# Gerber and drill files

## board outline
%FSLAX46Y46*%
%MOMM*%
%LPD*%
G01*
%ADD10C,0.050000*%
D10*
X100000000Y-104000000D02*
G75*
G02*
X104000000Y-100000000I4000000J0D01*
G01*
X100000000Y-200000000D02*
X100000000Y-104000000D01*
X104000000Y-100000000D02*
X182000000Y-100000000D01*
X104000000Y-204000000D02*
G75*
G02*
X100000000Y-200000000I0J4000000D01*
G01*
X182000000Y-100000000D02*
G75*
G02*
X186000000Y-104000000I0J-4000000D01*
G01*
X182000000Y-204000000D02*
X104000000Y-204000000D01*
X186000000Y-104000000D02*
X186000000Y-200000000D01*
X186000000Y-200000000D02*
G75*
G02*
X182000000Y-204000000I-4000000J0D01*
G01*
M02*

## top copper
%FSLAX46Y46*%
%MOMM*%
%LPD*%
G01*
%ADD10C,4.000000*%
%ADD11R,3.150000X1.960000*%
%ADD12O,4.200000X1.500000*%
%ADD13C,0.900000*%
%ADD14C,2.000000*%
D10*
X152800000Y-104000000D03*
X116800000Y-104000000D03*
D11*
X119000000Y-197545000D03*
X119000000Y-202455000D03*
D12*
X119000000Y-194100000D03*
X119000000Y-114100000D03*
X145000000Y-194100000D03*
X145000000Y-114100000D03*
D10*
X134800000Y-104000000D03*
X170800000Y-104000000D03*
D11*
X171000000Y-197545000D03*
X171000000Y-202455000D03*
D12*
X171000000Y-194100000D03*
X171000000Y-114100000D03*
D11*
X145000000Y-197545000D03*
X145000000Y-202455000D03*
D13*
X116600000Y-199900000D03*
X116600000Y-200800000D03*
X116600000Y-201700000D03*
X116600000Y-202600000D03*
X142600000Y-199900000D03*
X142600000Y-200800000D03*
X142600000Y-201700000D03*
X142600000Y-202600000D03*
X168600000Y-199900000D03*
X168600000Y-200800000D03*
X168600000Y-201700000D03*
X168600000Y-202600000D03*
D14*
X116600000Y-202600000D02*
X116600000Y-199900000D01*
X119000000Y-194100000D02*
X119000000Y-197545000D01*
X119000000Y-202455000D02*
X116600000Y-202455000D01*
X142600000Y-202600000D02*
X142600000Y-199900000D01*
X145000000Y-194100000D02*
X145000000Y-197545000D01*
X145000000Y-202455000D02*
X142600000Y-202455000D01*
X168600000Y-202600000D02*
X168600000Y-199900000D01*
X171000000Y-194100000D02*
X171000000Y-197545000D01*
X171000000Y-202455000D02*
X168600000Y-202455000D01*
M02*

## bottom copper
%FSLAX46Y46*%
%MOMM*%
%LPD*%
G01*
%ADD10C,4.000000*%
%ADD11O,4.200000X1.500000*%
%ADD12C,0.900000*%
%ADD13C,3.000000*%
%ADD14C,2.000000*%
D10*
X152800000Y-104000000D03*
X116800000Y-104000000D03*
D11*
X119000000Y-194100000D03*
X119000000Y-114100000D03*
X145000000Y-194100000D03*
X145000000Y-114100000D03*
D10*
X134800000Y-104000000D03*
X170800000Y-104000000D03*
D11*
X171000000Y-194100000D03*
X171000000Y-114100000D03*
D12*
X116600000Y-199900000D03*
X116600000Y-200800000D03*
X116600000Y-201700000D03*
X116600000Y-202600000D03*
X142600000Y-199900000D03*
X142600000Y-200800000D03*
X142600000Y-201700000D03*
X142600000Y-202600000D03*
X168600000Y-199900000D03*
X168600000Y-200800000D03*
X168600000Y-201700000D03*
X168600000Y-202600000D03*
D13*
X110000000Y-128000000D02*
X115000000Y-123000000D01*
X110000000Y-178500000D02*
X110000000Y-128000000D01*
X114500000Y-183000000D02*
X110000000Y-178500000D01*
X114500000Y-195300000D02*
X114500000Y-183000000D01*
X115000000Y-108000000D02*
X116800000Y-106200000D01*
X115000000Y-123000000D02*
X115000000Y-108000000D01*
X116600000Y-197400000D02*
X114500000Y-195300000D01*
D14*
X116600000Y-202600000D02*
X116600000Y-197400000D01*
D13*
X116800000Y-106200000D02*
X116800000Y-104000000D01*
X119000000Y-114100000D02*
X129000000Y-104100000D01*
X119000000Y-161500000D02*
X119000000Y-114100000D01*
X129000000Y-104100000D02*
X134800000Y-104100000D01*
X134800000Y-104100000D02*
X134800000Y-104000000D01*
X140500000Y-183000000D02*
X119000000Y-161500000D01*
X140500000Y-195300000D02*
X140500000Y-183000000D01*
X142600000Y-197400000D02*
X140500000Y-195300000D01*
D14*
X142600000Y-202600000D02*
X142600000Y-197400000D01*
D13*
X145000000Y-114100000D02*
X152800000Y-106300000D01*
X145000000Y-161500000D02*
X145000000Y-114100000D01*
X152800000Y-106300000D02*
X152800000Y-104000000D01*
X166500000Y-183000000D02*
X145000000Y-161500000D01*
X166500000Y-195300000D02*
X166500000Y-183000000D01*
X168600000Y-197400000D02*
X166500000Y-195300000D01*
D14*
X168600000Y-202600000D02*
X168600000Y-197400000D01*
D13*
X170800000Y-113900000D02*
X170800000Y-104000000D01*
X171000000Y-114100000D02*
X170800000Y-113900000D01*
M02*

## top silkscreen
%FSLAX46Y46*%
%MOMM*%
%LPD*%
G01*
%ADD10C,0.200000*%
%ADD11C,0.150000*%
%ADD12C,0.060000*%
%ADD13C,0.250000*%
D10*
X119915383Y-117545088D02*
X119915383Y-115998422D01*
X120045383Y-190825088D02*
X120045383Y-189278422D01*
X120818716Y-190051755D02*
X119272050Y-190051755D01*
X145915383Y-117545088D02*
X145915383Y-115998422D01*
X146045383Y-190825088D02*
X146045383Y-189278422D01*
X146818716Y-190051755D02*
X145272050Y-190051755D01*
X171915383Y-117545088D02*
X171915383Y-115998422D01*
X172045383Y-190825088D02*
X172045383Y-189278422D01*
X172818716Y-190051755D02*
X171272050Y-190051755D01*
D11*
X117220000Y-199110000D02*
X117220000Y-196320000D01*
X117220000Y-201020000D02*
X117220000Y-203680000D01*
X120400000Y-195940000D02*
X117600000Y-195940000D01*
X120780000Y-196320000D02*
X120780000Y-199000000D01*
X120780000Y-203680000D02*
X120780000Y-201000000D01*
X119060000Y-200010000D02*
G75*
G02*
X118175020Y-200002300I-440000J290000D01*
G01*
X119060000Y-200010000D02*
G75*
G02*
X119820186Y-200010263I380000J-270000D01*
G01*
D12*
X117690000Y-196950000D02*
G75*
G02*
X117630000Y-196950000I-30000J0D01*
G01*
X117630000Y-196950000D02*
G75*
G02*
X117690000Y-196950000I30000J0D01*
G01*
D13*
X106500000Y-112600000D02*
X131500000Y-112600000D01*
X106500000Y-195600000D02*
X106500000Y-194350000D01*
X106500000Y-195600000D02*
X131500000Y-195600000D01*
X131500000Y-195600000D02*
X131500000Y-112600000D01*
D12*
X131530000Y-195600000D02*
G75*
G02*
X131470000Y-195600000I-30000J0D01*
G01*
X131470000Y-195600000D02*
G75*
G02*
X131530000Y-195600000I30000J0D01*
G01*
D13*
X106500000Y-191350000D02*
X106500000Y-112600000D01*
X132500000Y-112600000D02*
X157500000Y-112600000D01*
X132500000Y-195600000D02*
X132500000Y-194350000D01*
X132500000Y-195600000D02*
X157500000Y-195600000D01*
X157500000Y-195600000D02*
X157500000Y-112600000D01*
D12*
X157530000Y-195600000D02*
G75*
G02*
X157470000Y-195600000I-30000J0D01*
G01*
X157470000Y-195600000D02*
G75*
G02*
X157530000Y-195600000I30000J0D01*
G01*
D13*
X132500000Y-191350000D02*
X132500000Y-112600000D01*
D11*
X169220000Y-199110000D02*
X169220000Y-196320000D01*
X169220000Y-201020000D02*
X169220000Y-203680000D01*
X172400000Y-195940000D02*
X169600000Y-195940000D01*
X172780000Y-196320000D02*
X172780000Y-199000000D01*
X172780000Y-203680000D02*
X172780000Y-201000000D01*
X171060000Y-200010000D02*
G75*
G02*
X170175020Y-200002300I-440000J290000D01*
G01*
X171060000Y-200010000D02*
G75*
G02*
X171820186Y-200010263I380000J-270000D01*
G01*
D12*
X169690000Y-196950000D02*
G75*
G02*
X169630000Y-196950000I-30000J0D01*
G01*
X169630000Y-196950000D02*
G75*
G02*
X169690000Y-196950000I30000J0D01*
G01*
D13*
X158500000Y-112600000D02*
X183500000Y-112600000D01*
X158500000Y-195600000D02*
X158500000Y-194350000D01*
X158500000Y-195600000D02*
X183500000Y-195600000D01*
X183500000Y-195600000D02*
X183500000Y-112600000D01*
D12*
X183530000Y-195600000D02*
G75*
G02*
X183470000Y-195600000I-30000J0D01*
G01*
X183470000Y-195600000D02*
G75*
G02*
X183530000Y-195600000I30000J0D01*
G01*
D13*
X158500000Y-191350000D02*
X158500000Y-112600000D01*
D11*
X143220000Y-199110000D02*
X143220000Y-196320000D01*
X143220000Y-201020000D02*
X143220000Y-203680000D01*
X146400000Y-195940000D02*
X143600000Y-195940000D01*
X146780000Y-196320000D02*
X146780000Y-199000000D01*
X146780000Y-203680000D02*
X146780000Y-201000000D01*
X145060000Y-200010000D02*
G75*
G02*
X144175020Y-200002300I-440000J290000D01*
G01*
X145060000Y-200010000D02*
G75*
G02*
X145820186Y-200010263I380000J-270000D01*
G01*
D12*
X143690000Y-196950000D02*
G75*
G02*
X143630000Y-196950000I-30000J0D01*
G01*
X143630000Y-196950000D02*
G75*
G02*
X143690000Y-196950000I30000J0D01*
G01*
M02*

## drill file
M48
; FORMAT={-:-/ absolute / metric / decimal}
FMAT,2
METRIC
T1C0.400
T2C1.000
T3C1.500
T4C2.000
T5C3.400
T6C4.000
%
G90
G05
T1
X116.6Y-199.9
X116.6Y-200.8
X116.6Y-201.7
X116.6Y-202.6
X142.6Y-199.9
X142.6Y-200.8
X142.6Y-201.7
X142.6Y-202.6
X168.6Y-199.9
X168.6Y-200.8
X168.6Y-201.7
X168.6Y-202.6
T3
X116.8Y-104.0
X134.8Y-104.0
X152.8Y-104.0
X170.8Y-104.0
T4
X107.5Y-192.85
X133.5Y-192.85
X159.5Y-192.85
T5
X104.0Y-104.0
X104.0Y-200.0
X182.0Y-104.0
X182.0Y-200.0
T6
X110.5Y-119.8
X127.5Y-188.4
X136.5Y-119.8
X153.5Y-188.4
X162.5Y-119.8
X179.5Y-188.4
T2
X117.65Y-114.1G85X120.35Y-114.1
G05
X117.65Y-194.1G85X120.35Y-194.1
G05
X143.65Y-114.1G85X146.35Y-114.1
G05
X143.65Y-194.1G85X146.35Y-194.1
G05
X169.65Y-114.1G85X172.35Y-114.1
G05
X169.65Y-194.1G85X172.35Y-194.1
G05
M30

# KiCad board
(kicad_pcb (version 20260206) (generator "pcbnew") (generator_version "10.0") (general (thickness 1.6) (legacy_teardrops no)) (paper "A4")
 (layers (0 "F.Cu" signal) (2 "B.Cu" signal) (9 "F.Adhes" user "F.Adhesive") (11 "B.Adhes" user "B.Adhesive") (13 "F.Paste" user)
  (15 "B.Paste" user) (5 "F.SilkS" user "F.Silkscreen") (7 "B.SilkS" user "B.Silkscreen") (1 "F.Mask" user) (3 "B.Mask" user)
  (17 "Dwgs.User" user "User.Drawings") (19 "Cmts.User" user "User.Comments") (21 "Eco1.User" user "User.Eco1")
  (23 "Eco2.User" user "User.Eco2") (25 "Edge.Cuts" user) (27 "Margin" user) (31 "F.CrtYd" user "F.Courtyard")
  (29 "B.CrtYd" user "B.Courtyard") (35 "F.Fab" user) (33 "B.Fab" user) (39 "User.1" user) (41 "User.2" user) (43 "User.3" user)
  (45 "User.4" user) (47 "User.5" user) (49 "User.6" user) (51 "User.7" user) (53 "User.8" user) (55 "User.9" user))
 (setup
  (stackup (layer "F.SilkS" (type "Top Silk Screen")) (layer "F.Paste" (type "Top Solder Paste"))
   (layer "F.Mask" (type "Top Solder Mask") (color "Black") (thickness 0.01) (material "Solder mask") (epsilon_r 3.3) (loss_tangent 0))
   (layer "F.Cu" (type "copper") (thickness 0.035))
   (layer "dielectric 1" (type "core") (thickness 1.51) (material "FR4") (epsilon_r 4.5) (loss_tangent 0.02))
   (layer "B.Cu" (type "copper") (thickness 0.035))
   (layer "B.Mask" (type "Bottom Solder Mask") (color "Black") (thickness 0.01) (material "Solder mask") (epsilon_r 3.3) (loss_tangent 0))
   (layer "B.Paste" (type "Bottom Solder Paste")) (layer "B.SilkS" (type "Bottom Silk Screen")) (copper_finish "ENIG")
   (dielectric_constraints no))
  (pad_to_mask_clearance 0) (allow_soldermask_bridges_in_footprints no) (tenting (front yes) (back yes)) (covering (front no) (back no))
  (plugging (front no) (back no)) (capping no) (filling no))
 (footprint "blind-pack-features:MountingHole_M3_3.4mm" (layer "F.Cu") (at 182 200)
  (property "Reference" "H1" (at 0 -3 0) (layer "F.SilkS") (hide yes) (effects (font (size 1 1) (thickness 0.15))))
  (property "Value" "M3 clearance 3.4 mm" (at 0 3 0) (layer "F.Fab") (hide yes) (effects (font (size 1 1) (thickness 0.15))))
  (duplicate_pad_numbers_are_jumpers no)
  (pad "" np_thru_hole circle (at 0 0) (size 3.4 3.4) (drill 3.4) (layers "*.Cu" "*.Mask")))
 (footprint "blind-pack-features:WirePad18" (layer "F.Cu") (at 152.8 104)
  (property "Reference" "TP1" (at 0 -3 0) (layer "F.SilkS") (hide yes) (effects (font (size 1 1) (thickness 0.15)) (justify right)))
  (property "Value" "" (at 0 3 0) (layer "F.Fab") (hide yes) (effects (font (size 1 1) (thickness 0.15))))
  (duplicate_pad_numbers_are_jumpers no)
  (pad "1" thru_hole circle (at 0 0) (size 4 4) (drill 1.5) (layers "*.Cu" "*.Mask") (remove_unused_layers no) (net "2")))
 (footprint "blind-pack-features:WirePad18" (layer "F.Cu") (at 116.8 104)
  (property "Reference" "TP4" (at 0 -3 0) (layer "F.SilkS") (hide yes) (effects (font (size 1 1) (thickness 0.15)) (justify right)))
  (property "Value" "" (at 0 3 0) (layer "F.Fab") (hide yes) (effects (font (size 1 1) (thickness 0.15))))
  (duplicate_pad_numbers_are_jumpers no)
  (pad "1" thru_hole circle (at 0 0) (size 4 4) (drill 1.5) (layers "*.Cu" "*.Mask") (remove_unused_layers no) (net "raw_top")))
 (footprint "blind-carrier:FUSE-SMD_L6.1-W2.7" (layer "F.Cu") (at 119 200 -90)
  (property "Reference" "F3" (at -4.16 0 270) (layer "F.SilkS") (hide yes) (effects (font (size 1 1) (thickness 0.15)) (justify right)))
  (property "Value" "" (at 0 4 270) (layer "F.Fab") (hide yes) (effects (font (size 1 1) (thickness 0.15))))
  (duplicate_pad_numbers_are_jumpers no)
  (fp_line (start -0.89 1.78) (end -3.68 1.78) (stroke (width 0.15) (type solid)) (layer "F.SilkS"))
  (fp_line (start 1.02 1.78) (end 3.68 1.78) (stroke (width 0.15) (type solid)) (layer "F.SilkS"))
  (fp_line (start -4.06 -1.4) (end -4.06 1.4) (stroke (width 0.15) (type solid)) (layer "F.SilkS"))
  (fp_line (start -3.68 -1.78) (end -1 -1.78) (stroke (width 0.15) (type solid)) (layer "F.SilkS"))
  (fp_line (start 3.68 -1.78) (end 1 -1.78) (stroke (width 0.15) (type solid)) (layer "F.SilkS"))
  (fp_arc (start 0.01 -0.06) (mid 0.246953 0.384585) (end 0.0023 0.82498) (stroke (width 0.15) (type solid)) (layer "F.SilkS"))
  (fp_arc (start 0.01 -0.06) (mid -0.186154 -0.440161) (end 0.010263 -0.820186) (stroke (width 0.15) (type solid)) (layer "F.SilkS"))
  (fp_circle (center -3.05 1.34) (end -3.02 1.34) (stroke (width 0.06) (type solid)) (fill no) (layer "F.SilkS"))
  (pad "1" smd rect (at -2.455 0 270) (size 1.96 3.15) (layers "F.Cu" "F.Mask" "F.Paste") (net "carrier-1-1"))
  (pad "2" smd rect (at 2.455 0 270) (size 1.96 3.15) (layers "F.Cu" "F.Mask" "F.Paste") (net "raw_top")))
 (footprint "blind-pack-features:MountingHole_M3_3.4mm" (layer "F.Cu") (at 104 200)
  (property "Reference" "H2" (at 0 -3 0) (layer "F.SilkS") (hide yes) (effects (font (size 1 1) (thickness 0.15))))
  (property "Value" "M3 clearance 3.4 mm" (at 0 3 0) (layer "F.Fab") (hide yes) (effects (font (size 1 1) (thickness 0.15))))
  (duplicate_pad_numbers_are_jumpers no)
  (pad "" np_thru_hole circle (at 0 0) (size 3.4 3.4) (drill 3.4) (layers "*.Cu" "*.Mask")))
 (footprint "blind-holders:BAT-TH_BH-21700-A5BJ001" (layer "F.Cu") (at 119 154.1 90)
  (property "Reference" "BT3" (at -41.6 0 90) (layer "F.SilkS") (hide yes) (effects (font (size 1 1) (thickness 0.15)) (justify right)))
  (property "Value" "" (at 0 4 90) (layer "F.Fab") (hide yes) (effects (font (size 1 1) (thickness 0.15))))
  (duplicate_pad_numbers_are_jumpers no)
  (fp_line (start 41.5 -12.5) (end 41.5 12.5) (stroke (width 0.25) (type solid)) (layer "F.SilkS"))
  (fp_line (start -41.5 -12.5) (end -40.25 -12.5) (stroke (width 0.25) (type solid)) (layer "F.SilkS"))
  (fp_line (start -41.5 -12.5) (end -41.5 12.5) (stroke (width 0.25) (type solid)) (layer "F.SilkS"))
  (fp_line (start -41.5 12.5) (end 41.5 12.5) (stroke (width 0.25) (type solid)) (layer "F.SilkS"))
  (fp_circle (center -41.5 12.5) (end -41.47 12.5) (stroke (width 0.06) (type solid)) (fill no) (layer "F.SilkS"))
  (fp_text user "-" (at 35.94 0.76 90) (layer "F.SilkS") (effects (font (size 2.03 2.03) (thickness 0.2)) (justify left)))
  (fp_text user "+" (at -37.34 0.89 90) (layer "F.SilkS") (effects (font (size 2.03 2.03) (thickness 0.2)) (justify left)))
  (pad "" np_thru_hole circle (at -38.75 -11.5 90) (size 2 2) (drill 2) (layers "*.Cu" "*.Mask"))
  (pad "" np_thru_hole circle (at -34.3 8.5 90) (size 4 4) (drill 4) (layers "*.Cu" "*.Mask"))
  (pad "" np_thru_hole circle (at 34.3 -8.5 90) (size 4 4) (drill 4) (layers "*.Cu" "*.Mask"))
  (pad "1" thru_hole oval (at -40 0 90) (size 1.5 4.2) (drill oval 1 3.7) (layers "*.Cu" "*.Mask") (remove_unused_layers no)
   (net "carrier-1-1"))
  (pad "2" thru_hole oval (at 40 0 90) (size 1.5 4.2) (drill oval 1 3.7) (layers "*.Cu" "*.Mask") (remove_unused_layers no)
   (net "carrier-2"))
  (fp_line (start -37.25 -12.5) (end 41.5 -12.5) (stroke (width 0.25) (type solid)) (layer "F.SilkS")))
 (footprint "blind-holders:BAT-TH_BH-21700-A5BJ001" (layer "F.Cu") (at 145 154.1 90)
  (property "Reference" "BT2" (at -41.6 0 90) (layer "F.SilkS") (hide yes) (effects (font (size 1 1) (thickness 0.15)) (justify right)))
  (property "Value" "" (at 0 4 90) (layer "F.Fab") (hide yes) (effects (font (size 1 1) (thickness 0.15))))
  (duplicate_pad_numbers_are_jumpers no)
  (fp_line (start 41.5 -12.5) (end 41.5 12.5) (stroke (width 0.25) (type solid)) (layer "F.SilkS"))
  (fp_line (start -41.5 -12.5) (end -40.25 -12.5) (stroke (width 0.25) (type solid)) (layer "F.SilkS"))
  (fp_line (start -41.5 -12.5) (end -41.5 12.5) (stroke (width 0.25) (type solid)) (layer "F.SilkS"))
  (fp_line (start -41.5 12.5) (end 41.5 12.5) (stroke (width 0.25) (type solid)) (layer "F.SilkS"))
  (fp_circle (center -41.5 12.5) (end -41.47 12.5) (stroke (width 0.06) (type solid)) (fill no) (layer "F.SilkS"))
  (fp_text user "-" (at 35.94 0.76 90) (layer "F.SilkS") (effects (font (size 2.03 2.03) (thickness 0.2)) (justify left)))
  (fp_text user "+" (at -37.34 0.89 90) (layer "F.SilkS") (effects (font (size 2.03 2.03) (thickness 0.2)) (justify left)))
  (pad "" np_thru_hole circle (at -38.75 -11.5 90) (size 2 2) (drill 2) (layers "*.Cu" "*.Mask"))
  (pad "" np_thru_hole circle (at -34.3 8.5 90) (size 4 4) (drill 4) (layers "*.Cu" "*.Mask"))
  (pad "" np_thru_hole circle (at 34.3 -8.5 90) (size 4 4) (drill 4) (layers "*.Cu" "*.Mask"))
  (pad "1" thru_hole oval (at -40 0 90) (size 1.5 4.2) (drill oval 1 3.7) (layers "*.Cu" "*.Mask") (remove_unused_layers no)
   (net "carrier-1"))
  (pad "2" thru_hole oval (at 40 0 90) (size 1.5 4.2) (drill oval 1 3.7) (layers "*.Cu" "*.Mask") (remove_unused_layers no) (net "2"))
  (fp_line (start -37.25 -12.5) (end 41.5 -12.5) (stroke (width 0.25) (type solid)) (layer "F.SilkS")))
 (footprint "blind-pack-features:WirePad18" (layer "F.Cu") (at 134.8 104)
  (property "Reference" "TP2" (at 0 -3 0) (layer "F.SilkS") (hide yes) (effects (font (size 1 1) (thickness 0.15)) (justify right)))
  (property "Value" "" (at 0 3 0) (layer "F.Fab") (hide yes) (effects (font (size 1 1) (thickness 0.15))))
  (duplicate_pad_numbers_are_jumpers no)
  (pad "1" thru_hole circle (at 0 0) (size 4 4) (drill 1.5) (layers "*.Cu" "*.Mask") (remove_unused_layers no) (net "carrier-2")))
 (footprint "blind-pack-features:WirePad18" (layer "F.Cu") (at 170.8 104)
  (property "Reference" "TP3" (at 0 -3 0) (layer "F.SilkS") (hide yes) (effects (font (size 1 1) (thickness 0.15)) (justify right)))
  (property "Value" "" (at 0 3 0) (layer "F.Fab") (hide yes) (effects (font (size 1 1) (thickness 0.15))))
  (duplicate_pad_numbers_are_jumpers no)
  (pad "1" thru_hole circle (at 0 0) (size 4 4) (drill 1.5) (layers "*.Cu" "*.Mask") (remove_unused_layers no) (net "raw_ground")))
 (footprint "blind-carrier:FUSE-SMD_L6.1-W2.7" (layer "F.Cu") (at 171 200 -90)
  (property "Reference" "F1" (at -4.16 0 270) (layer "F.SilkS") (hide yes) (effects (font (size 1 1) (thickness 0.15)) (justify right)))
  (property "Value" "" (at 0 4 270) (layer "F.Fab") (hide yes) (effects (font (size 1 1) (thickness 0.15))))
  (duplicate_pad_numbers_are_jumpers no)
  (fp_line (start -0.89 1.78) (end -3.68 1.78) (stroke (width 0.15) (type solid)) (layer "F.SilkS"))
  (fp_line (start 1.02 1.78) (end 3.68 1.78) (stroke (width 0.15) (type solid)) (layer "F.SilkS"))
  (fp_line (start -4.06 -1.4) (end -4.06 1.4) (stroke (width 0.15) (type solid)) (layer "F.SilkS"))
  (fp_line (start -3.68 -1.78) (end -1 -1.78) (stroke (width 0.15) (type solid)) (layer "F.SilkS"))
  (fp_line (start 3.68 -1.78) (end 1 -1.78) (stroke (width 0.15) (type solid)) (layer "F.SilkS"))
  (fp_arc (start 0.01 -0.06) (mid 0.246953 0.384585) (end 0.0023 0.82498) (stroke (width 0.15) (type solid)) (layer "F.SilkS"))
  (fp_arc (start 0.01 -0.06) (mid -0.186154 -0.440161) (end 0.010263 -0.820186) (stroke (width 0.15) (type solid)) (layer "F.SilkS"))
  (fp_circle (center -3.05 1.34) (end -3.02 1.34) (stroke (width 0.06) (type solid)) (fill no) (layer "F.SilkS"))
  (pad "1" smd rect (at -2.455 0 270) (size 1.96 3.15) (layers "F.Cu" "F.Mask" "F.Paste") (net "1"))
  (pad "2" smd rect (at 2.455 0 270) (size 1.96 3.15) (layers "F.Cu" "F.Mask" "F.Paste") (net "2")))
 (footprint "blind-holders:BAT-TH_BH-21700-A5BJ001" (layer "F.Cu") (at 171 154.1 90)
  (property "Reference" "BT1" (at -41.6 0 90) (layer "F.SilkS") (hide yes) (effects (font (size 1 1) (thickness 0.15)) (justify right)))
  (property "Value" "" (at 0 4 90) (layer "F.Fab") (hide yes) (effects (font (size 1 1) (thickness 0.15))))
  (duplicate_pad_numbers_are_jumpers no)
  (fp_line (start 41.5 -12.5) (end 41.5 12.5) (stroke (width 0.25) (type solid)) (layer "F.SilkS"))
  (fp_line (start -41.5 -12.5) (end -40.25 -12.5) (stroke (width 0.25) (type solid)) (layer "F.SilkS"))
  (fp_line (start -41.5 -12.5) (end -41.5 12.5) (stroke (width 0.25) (type solid)) (layer "F.SilkS"))
  (fp_line (start -41.5 12.5) (end 41.5 12.5) (stroke (width 0.25) (type solid)) (layer "F.SilkS"))
  (fp_circle (center -41.5 12.5) (end -41.47 12.5) (stroke (width 0.06) (type solid)) (fill no) (layer "F.SilkS"))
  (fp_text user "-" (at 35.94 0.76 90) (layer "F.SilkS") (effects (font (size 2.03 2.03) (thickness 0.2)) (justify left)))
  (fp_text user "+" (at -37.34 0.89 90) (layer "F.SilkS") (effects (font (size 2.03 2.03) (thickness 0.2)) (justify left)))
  (pad "" np_thru_hole circle (at -38.75 -11.5 90) (size 2 2) (drill 2) (layers "*.Cu" "*.Mask"))
  (pad "" np_thru_hole circle (at -34.3 8.5 90) (size 4 4) (drill 4) (layers "*.Cu" "*.Mask"))
  (pad "" np_thru_hole circle (at 34.3 -8.5 90) (size 4 4) (drill 4) (layers "*.Cu" "*.Mask"))
  (pad "1" thru_hole oval (at -40 0 90) (size 1.5 4.2) (drill oval 1 3.7) (layers "*.Cu" "*.Mask") (remove_unused_layers no) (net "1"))
  (pad "2" thru_hole oval (at 40 0 90) (size 1.5 4.2) (drill oval 1 3.7) (layers "*.Cu" "*.Mask") (remove_unused_layers no)
   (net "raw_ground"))
  (fp_line (start -37.25 -12.5) (end 41.5 -12.5) (stroke (width 0.25) (type solid)) (layer "F.SilkS")))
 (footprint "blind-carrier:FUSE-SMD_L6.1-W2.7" (layer "F.Cu") (at 145 200 -90)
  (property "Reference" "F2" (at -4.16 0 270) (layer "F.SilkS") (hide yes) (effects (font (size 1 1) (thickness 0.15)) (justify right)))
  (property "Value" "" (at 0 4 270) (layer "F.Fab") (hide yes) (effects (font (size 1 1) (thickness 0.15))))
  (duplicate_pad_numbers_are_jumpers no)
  (fp_line (start -0.89 1.78) (end -3.68 1.78) (stroke (width 0.15) (type solid)) (layer "F.SilkS"))
  (fp_line (start 1.02 1.78) (end 3.68 1.78) (stroke (width 0.15) (type solid)) (layer "F.SilkS"))
  (fp_line (start -4.06 -1.4) (end -4.06 1.4) (stroke (width 0.15) (type solid)) (layer "F.SilkS"))
  (fp_line (start -3.68 -1.78) (end -1 -1.78) (stroke (width 0.15) (type solid)) (layer "F.SilkS"))
  (fp_line (start 3.68 -1.78) (end 1 -1.78) (stroke (width 0.15) (type solid)) (layer "F.SilkS"))
  (fp_arc (start 0.01 -0.06) (mid 0.246953 0.384585) (end 0.0023 0.82498) (stroke (width 0.15) (type solid)) (layer "F.SilkS"))
  (fp_arc (start 0.01 -0.06) (mid -0.186154 -0.440161) (end 0.010263 -0.820186) (stroke (width 0.15) (type solid)) (layer "F.SilkS"))
  (fp_circle (center -3.05 1.34) (end -3.02 1.34) (stroke (width 0.06) (type solid)) (fill no) (layer "F.SilkS"))
  (pad "1" smd rect (at -2.455 0 270) (size 1.96 3.15) (layers "F.Cu" "F.Mask" "F.Paste") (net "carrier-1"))
  (pad "2" smd rect (at 2.455 0 270) (size 1.96 3.15) (layers "F.Cu" "F.Mask" "F.Paste") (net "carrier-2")))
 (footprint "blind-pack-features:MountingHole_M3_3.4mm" (layer "F.Cu") (at 182 104)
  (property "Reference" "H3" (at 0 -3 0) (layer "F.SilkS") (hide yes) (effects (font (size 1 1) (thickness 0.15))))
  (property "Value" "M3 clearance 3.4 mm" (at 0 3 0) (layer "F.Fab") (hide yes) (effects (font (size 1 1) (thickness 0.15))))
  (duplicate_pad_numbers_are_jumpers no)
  (pad "" np_thru_hole circle (at 0 0) (size 3.4 3.4) (drill 3.4) (layers "*.Cu" "*.Mask")))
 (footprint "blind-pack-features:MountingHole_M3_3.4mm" (layer "F.Cu") (at 104 104)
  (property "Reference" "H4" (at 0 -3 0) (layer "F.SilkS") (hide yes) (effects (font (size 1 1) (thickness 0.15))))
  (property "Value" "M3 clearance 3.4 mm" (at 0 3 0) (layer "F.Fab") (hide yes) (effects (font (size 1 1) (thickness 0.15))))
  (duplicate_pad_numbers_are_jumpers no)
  (pad "" np_thru_hole circle (at 0 0) (size 3.4 3.4) (drill 3.4) (layers "*.Cu" "*.Mask")))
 (gr_arc (start 100 104) (mid 101.171572 101.171572) (end 104 100) (stroke (width 0.05) (type default)) (layer "Edge.Cuts"))
 (gr_line (start 100 200) (end 100 104) (stroke (width 0.05) (type default)) (layer "Edge.Cuts"))
 (gr_line (start 104 100) (end 182 100) (stroke (width 0.05) (type default)) (layer "Edge.Cuts"))
 (gr_arc (start 104 204) (mid 101.171572 202.828427) (end 100 200) (stroke (width 0.05) (type default)) (layer "Edge.Cuts"))
 (gr_arc (start 182 100) (mid 184.828427 101.171572) (end 186 104) (stroke (width 0.05) (type default)) (layer "Edge.Cuts"))
 (gr_line (start 182 204) (end 104 204) (stroke (width 0.05) (type default)) (layer "Edge.Cuts"))
 (gr_line (start 186 104) (end 186 200) (stroke (width 0.05) (type default)) (layer "Edge.Cuts"))
 (gr_arc (start 186 200) (mid 184.828427 202.828427) (end 182 204) (stroke (width 0.05) (type default)) (layer "Edge.Cuts"))
 (segment (start 110 128) (end 115 123) (width 3) (layer "B.Cu") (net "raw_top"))
 (segment (start 110 178.5) (end 110 128) (width 3) (layer "B.Cu") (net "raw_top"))
 (via (at 116.6 199.9) (size 0.9) (drill 0.4) (layers "F.Cu" "B.Cu") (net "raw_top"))
 (via (at 116.6 200.8) (size 0.9) (drill 0.4) (layers "F.Cu" "B.Cu") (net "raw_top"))
 (via (at 116.6 201.7) (size 0.9) (drill 0.4) (layers "F.Cu" "B.Cu") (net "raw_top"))
 (via (at 116.6 202.6) (size 0.9) (drill 0.4) (layers "F.Cu" "B.Cu") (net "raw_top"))
 (segment (start 114.5 183) (end 110 178.5) (width 3) (layer "B.Cu") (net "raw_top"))
 (segment (start 114.5 195.3) (end 114.5 183) (width 3) (layer "B.Cu") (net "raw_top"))
 (segment (start 115 108) (end 116.8 106.2) (width 3) (layer "B.Cu") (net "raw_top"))
 (segment (start 115 123) (end 115 108) (width 3) (layer "B.Cu") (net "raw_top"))
 (segment (start 116.6 197.4) (end 114.5 195.3) (width 3) (layer "B.Cu") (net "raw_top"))
 (segment (start 116.6 202.6) (end 116.6 197.4) (width 2) (layer "B.Cu") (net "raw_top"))
 (segment (start 116.6 202.6) (end 116.6 199.9) (width 2) (layer "F.Cu") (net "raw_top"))
 (segment (start 116.8 106.2) (end 116.8 104) (width 3) (layer "B.Cu") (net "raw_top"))
 (segment (start 119 114.1) (end 129 104.1) (width 3) (layer "B.Cu") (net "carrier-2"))
 (via (at 142.6 199.9) (size 0.9) (drill 0.4) (layers "F.Cu" "B.Cu") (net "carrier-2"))
 (via (at 142.6 200.8) (size 0.9) (drill 0.4) (layers "F.Cu" "B.Cu") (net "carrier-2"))
 (via (at 142.6 201.7) (size 0.9) (drill 0.4) (layers "F.Cu" "B.Cu") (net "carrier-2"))
 (via (at 142.6 202.6) (size 0.9) (drill 0.4) (layers "F.Cu" "B.Cu") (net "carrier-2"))
 (segment (start 119 161.5) (end 119 114.1) (width 3) (layer "B.Cu") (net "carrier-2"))
 (segment (start 119 194.1) (end 119 197.545) (width 2) (layer "F.Cu") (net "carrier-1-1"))
 (segment (start 119 202.455) (end 116.6 202.455) (width 2) (layer "F.Cu") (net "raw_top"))
 (segment (start 129 104.1) (end 134.8 104.1) (width 3) (layer "B.Cu") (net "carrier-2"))
 (segment (start 134.8 104.1) (end 134.8 104) (width 3) (layer "B.Cu") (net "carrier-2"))
 (segment (start 140.5 183) (end 119 161.5) (width 3) (layer "B.Cu") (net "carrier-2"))
 (segment (start 140.5 195.3) (end 140.5 183) (width 3) (layer "B.Cu") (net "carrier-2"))
 (segment (start 142.6 197.4) (end 140.5 195.3) (width 3) (layer "B.Cu") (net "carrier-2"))
 (segment (start 142.6 202.6) (end 142.6 197.4) (width 2) (layer "B.Cu") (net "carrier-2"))
 (segment (start 142.6 202.6) (end 142.6 199.9) (width 2) (layer "F.Cu") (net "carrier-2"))
 (segment (start 145 114.1) (end 152.8 106.3) (width 3) (layer "B.Cu") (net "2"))
 (segment (start 145 161.5) (end 145 114.1) (width 3) (layer "B.Cu") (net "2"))
 (segment (start 145 194.1) (end 145 197.545) (width 2) (layer "F.Cu") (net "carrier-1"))
 (segment (start 145 202.455) (end 142.6 202.455) (width 2) (layer "F.Cu") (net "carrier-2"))
 (segment (start 152.8 106.3) (end 152.8 104) (width 3) (layer "B.Cu") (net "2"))
 (segment (start 166.5 183) (end 145 161.5) (width 3) (layer "B.Cu") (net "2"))
 (via (at 168.6 199.9) (size 0.9) (drill 0.4) (layers "F.Cu" "B.Cu") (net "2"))
 (via (at 168.6 200.8) (size 0.9) (drill 0.4) (layers "F.Cu" "B.Cu") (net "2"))
 (via (at 168.6 201.7) (size 0.9) (drill 0.4) (layers "F.Cu" "B.Cu") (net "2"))
 (via (at 168.6 202.6) (size 0.9) (drill 0.4) (layers "F.Cu" "B.Cu") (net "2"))
 (segment (start 166.5 195.3) (end 166.5 183) (width 3) (layer "B.Cu") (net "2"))
 (segment (start 168.6 197.4) (end 166.5 195.3) (width 3) (layer "B.Cu") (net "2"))
 (segment (start 168.6 202.6) (end 168.6 197.4) (width 2) (layer "B.Cu") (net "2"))
 (segment (start 168.6 202.6) (end 168.6 199.9) (width 2) (layer "F.Cu") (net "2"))
 (segment (start 170.8 113.9) (end 170.8 104) (width 3) (layer "B.Cu") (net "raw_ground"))
 (segment (start 171 114.1) (end 170.8 113.9) (width 3) (layer "B.Cu") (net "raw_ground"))
 (segment (start 171 194.1) (end 171 197.545) (width 2) (layer "F.Cu") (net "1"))
 (segment (start 171 202.455) (end 168.6 202.455) (width 2) (layer "F.Cu") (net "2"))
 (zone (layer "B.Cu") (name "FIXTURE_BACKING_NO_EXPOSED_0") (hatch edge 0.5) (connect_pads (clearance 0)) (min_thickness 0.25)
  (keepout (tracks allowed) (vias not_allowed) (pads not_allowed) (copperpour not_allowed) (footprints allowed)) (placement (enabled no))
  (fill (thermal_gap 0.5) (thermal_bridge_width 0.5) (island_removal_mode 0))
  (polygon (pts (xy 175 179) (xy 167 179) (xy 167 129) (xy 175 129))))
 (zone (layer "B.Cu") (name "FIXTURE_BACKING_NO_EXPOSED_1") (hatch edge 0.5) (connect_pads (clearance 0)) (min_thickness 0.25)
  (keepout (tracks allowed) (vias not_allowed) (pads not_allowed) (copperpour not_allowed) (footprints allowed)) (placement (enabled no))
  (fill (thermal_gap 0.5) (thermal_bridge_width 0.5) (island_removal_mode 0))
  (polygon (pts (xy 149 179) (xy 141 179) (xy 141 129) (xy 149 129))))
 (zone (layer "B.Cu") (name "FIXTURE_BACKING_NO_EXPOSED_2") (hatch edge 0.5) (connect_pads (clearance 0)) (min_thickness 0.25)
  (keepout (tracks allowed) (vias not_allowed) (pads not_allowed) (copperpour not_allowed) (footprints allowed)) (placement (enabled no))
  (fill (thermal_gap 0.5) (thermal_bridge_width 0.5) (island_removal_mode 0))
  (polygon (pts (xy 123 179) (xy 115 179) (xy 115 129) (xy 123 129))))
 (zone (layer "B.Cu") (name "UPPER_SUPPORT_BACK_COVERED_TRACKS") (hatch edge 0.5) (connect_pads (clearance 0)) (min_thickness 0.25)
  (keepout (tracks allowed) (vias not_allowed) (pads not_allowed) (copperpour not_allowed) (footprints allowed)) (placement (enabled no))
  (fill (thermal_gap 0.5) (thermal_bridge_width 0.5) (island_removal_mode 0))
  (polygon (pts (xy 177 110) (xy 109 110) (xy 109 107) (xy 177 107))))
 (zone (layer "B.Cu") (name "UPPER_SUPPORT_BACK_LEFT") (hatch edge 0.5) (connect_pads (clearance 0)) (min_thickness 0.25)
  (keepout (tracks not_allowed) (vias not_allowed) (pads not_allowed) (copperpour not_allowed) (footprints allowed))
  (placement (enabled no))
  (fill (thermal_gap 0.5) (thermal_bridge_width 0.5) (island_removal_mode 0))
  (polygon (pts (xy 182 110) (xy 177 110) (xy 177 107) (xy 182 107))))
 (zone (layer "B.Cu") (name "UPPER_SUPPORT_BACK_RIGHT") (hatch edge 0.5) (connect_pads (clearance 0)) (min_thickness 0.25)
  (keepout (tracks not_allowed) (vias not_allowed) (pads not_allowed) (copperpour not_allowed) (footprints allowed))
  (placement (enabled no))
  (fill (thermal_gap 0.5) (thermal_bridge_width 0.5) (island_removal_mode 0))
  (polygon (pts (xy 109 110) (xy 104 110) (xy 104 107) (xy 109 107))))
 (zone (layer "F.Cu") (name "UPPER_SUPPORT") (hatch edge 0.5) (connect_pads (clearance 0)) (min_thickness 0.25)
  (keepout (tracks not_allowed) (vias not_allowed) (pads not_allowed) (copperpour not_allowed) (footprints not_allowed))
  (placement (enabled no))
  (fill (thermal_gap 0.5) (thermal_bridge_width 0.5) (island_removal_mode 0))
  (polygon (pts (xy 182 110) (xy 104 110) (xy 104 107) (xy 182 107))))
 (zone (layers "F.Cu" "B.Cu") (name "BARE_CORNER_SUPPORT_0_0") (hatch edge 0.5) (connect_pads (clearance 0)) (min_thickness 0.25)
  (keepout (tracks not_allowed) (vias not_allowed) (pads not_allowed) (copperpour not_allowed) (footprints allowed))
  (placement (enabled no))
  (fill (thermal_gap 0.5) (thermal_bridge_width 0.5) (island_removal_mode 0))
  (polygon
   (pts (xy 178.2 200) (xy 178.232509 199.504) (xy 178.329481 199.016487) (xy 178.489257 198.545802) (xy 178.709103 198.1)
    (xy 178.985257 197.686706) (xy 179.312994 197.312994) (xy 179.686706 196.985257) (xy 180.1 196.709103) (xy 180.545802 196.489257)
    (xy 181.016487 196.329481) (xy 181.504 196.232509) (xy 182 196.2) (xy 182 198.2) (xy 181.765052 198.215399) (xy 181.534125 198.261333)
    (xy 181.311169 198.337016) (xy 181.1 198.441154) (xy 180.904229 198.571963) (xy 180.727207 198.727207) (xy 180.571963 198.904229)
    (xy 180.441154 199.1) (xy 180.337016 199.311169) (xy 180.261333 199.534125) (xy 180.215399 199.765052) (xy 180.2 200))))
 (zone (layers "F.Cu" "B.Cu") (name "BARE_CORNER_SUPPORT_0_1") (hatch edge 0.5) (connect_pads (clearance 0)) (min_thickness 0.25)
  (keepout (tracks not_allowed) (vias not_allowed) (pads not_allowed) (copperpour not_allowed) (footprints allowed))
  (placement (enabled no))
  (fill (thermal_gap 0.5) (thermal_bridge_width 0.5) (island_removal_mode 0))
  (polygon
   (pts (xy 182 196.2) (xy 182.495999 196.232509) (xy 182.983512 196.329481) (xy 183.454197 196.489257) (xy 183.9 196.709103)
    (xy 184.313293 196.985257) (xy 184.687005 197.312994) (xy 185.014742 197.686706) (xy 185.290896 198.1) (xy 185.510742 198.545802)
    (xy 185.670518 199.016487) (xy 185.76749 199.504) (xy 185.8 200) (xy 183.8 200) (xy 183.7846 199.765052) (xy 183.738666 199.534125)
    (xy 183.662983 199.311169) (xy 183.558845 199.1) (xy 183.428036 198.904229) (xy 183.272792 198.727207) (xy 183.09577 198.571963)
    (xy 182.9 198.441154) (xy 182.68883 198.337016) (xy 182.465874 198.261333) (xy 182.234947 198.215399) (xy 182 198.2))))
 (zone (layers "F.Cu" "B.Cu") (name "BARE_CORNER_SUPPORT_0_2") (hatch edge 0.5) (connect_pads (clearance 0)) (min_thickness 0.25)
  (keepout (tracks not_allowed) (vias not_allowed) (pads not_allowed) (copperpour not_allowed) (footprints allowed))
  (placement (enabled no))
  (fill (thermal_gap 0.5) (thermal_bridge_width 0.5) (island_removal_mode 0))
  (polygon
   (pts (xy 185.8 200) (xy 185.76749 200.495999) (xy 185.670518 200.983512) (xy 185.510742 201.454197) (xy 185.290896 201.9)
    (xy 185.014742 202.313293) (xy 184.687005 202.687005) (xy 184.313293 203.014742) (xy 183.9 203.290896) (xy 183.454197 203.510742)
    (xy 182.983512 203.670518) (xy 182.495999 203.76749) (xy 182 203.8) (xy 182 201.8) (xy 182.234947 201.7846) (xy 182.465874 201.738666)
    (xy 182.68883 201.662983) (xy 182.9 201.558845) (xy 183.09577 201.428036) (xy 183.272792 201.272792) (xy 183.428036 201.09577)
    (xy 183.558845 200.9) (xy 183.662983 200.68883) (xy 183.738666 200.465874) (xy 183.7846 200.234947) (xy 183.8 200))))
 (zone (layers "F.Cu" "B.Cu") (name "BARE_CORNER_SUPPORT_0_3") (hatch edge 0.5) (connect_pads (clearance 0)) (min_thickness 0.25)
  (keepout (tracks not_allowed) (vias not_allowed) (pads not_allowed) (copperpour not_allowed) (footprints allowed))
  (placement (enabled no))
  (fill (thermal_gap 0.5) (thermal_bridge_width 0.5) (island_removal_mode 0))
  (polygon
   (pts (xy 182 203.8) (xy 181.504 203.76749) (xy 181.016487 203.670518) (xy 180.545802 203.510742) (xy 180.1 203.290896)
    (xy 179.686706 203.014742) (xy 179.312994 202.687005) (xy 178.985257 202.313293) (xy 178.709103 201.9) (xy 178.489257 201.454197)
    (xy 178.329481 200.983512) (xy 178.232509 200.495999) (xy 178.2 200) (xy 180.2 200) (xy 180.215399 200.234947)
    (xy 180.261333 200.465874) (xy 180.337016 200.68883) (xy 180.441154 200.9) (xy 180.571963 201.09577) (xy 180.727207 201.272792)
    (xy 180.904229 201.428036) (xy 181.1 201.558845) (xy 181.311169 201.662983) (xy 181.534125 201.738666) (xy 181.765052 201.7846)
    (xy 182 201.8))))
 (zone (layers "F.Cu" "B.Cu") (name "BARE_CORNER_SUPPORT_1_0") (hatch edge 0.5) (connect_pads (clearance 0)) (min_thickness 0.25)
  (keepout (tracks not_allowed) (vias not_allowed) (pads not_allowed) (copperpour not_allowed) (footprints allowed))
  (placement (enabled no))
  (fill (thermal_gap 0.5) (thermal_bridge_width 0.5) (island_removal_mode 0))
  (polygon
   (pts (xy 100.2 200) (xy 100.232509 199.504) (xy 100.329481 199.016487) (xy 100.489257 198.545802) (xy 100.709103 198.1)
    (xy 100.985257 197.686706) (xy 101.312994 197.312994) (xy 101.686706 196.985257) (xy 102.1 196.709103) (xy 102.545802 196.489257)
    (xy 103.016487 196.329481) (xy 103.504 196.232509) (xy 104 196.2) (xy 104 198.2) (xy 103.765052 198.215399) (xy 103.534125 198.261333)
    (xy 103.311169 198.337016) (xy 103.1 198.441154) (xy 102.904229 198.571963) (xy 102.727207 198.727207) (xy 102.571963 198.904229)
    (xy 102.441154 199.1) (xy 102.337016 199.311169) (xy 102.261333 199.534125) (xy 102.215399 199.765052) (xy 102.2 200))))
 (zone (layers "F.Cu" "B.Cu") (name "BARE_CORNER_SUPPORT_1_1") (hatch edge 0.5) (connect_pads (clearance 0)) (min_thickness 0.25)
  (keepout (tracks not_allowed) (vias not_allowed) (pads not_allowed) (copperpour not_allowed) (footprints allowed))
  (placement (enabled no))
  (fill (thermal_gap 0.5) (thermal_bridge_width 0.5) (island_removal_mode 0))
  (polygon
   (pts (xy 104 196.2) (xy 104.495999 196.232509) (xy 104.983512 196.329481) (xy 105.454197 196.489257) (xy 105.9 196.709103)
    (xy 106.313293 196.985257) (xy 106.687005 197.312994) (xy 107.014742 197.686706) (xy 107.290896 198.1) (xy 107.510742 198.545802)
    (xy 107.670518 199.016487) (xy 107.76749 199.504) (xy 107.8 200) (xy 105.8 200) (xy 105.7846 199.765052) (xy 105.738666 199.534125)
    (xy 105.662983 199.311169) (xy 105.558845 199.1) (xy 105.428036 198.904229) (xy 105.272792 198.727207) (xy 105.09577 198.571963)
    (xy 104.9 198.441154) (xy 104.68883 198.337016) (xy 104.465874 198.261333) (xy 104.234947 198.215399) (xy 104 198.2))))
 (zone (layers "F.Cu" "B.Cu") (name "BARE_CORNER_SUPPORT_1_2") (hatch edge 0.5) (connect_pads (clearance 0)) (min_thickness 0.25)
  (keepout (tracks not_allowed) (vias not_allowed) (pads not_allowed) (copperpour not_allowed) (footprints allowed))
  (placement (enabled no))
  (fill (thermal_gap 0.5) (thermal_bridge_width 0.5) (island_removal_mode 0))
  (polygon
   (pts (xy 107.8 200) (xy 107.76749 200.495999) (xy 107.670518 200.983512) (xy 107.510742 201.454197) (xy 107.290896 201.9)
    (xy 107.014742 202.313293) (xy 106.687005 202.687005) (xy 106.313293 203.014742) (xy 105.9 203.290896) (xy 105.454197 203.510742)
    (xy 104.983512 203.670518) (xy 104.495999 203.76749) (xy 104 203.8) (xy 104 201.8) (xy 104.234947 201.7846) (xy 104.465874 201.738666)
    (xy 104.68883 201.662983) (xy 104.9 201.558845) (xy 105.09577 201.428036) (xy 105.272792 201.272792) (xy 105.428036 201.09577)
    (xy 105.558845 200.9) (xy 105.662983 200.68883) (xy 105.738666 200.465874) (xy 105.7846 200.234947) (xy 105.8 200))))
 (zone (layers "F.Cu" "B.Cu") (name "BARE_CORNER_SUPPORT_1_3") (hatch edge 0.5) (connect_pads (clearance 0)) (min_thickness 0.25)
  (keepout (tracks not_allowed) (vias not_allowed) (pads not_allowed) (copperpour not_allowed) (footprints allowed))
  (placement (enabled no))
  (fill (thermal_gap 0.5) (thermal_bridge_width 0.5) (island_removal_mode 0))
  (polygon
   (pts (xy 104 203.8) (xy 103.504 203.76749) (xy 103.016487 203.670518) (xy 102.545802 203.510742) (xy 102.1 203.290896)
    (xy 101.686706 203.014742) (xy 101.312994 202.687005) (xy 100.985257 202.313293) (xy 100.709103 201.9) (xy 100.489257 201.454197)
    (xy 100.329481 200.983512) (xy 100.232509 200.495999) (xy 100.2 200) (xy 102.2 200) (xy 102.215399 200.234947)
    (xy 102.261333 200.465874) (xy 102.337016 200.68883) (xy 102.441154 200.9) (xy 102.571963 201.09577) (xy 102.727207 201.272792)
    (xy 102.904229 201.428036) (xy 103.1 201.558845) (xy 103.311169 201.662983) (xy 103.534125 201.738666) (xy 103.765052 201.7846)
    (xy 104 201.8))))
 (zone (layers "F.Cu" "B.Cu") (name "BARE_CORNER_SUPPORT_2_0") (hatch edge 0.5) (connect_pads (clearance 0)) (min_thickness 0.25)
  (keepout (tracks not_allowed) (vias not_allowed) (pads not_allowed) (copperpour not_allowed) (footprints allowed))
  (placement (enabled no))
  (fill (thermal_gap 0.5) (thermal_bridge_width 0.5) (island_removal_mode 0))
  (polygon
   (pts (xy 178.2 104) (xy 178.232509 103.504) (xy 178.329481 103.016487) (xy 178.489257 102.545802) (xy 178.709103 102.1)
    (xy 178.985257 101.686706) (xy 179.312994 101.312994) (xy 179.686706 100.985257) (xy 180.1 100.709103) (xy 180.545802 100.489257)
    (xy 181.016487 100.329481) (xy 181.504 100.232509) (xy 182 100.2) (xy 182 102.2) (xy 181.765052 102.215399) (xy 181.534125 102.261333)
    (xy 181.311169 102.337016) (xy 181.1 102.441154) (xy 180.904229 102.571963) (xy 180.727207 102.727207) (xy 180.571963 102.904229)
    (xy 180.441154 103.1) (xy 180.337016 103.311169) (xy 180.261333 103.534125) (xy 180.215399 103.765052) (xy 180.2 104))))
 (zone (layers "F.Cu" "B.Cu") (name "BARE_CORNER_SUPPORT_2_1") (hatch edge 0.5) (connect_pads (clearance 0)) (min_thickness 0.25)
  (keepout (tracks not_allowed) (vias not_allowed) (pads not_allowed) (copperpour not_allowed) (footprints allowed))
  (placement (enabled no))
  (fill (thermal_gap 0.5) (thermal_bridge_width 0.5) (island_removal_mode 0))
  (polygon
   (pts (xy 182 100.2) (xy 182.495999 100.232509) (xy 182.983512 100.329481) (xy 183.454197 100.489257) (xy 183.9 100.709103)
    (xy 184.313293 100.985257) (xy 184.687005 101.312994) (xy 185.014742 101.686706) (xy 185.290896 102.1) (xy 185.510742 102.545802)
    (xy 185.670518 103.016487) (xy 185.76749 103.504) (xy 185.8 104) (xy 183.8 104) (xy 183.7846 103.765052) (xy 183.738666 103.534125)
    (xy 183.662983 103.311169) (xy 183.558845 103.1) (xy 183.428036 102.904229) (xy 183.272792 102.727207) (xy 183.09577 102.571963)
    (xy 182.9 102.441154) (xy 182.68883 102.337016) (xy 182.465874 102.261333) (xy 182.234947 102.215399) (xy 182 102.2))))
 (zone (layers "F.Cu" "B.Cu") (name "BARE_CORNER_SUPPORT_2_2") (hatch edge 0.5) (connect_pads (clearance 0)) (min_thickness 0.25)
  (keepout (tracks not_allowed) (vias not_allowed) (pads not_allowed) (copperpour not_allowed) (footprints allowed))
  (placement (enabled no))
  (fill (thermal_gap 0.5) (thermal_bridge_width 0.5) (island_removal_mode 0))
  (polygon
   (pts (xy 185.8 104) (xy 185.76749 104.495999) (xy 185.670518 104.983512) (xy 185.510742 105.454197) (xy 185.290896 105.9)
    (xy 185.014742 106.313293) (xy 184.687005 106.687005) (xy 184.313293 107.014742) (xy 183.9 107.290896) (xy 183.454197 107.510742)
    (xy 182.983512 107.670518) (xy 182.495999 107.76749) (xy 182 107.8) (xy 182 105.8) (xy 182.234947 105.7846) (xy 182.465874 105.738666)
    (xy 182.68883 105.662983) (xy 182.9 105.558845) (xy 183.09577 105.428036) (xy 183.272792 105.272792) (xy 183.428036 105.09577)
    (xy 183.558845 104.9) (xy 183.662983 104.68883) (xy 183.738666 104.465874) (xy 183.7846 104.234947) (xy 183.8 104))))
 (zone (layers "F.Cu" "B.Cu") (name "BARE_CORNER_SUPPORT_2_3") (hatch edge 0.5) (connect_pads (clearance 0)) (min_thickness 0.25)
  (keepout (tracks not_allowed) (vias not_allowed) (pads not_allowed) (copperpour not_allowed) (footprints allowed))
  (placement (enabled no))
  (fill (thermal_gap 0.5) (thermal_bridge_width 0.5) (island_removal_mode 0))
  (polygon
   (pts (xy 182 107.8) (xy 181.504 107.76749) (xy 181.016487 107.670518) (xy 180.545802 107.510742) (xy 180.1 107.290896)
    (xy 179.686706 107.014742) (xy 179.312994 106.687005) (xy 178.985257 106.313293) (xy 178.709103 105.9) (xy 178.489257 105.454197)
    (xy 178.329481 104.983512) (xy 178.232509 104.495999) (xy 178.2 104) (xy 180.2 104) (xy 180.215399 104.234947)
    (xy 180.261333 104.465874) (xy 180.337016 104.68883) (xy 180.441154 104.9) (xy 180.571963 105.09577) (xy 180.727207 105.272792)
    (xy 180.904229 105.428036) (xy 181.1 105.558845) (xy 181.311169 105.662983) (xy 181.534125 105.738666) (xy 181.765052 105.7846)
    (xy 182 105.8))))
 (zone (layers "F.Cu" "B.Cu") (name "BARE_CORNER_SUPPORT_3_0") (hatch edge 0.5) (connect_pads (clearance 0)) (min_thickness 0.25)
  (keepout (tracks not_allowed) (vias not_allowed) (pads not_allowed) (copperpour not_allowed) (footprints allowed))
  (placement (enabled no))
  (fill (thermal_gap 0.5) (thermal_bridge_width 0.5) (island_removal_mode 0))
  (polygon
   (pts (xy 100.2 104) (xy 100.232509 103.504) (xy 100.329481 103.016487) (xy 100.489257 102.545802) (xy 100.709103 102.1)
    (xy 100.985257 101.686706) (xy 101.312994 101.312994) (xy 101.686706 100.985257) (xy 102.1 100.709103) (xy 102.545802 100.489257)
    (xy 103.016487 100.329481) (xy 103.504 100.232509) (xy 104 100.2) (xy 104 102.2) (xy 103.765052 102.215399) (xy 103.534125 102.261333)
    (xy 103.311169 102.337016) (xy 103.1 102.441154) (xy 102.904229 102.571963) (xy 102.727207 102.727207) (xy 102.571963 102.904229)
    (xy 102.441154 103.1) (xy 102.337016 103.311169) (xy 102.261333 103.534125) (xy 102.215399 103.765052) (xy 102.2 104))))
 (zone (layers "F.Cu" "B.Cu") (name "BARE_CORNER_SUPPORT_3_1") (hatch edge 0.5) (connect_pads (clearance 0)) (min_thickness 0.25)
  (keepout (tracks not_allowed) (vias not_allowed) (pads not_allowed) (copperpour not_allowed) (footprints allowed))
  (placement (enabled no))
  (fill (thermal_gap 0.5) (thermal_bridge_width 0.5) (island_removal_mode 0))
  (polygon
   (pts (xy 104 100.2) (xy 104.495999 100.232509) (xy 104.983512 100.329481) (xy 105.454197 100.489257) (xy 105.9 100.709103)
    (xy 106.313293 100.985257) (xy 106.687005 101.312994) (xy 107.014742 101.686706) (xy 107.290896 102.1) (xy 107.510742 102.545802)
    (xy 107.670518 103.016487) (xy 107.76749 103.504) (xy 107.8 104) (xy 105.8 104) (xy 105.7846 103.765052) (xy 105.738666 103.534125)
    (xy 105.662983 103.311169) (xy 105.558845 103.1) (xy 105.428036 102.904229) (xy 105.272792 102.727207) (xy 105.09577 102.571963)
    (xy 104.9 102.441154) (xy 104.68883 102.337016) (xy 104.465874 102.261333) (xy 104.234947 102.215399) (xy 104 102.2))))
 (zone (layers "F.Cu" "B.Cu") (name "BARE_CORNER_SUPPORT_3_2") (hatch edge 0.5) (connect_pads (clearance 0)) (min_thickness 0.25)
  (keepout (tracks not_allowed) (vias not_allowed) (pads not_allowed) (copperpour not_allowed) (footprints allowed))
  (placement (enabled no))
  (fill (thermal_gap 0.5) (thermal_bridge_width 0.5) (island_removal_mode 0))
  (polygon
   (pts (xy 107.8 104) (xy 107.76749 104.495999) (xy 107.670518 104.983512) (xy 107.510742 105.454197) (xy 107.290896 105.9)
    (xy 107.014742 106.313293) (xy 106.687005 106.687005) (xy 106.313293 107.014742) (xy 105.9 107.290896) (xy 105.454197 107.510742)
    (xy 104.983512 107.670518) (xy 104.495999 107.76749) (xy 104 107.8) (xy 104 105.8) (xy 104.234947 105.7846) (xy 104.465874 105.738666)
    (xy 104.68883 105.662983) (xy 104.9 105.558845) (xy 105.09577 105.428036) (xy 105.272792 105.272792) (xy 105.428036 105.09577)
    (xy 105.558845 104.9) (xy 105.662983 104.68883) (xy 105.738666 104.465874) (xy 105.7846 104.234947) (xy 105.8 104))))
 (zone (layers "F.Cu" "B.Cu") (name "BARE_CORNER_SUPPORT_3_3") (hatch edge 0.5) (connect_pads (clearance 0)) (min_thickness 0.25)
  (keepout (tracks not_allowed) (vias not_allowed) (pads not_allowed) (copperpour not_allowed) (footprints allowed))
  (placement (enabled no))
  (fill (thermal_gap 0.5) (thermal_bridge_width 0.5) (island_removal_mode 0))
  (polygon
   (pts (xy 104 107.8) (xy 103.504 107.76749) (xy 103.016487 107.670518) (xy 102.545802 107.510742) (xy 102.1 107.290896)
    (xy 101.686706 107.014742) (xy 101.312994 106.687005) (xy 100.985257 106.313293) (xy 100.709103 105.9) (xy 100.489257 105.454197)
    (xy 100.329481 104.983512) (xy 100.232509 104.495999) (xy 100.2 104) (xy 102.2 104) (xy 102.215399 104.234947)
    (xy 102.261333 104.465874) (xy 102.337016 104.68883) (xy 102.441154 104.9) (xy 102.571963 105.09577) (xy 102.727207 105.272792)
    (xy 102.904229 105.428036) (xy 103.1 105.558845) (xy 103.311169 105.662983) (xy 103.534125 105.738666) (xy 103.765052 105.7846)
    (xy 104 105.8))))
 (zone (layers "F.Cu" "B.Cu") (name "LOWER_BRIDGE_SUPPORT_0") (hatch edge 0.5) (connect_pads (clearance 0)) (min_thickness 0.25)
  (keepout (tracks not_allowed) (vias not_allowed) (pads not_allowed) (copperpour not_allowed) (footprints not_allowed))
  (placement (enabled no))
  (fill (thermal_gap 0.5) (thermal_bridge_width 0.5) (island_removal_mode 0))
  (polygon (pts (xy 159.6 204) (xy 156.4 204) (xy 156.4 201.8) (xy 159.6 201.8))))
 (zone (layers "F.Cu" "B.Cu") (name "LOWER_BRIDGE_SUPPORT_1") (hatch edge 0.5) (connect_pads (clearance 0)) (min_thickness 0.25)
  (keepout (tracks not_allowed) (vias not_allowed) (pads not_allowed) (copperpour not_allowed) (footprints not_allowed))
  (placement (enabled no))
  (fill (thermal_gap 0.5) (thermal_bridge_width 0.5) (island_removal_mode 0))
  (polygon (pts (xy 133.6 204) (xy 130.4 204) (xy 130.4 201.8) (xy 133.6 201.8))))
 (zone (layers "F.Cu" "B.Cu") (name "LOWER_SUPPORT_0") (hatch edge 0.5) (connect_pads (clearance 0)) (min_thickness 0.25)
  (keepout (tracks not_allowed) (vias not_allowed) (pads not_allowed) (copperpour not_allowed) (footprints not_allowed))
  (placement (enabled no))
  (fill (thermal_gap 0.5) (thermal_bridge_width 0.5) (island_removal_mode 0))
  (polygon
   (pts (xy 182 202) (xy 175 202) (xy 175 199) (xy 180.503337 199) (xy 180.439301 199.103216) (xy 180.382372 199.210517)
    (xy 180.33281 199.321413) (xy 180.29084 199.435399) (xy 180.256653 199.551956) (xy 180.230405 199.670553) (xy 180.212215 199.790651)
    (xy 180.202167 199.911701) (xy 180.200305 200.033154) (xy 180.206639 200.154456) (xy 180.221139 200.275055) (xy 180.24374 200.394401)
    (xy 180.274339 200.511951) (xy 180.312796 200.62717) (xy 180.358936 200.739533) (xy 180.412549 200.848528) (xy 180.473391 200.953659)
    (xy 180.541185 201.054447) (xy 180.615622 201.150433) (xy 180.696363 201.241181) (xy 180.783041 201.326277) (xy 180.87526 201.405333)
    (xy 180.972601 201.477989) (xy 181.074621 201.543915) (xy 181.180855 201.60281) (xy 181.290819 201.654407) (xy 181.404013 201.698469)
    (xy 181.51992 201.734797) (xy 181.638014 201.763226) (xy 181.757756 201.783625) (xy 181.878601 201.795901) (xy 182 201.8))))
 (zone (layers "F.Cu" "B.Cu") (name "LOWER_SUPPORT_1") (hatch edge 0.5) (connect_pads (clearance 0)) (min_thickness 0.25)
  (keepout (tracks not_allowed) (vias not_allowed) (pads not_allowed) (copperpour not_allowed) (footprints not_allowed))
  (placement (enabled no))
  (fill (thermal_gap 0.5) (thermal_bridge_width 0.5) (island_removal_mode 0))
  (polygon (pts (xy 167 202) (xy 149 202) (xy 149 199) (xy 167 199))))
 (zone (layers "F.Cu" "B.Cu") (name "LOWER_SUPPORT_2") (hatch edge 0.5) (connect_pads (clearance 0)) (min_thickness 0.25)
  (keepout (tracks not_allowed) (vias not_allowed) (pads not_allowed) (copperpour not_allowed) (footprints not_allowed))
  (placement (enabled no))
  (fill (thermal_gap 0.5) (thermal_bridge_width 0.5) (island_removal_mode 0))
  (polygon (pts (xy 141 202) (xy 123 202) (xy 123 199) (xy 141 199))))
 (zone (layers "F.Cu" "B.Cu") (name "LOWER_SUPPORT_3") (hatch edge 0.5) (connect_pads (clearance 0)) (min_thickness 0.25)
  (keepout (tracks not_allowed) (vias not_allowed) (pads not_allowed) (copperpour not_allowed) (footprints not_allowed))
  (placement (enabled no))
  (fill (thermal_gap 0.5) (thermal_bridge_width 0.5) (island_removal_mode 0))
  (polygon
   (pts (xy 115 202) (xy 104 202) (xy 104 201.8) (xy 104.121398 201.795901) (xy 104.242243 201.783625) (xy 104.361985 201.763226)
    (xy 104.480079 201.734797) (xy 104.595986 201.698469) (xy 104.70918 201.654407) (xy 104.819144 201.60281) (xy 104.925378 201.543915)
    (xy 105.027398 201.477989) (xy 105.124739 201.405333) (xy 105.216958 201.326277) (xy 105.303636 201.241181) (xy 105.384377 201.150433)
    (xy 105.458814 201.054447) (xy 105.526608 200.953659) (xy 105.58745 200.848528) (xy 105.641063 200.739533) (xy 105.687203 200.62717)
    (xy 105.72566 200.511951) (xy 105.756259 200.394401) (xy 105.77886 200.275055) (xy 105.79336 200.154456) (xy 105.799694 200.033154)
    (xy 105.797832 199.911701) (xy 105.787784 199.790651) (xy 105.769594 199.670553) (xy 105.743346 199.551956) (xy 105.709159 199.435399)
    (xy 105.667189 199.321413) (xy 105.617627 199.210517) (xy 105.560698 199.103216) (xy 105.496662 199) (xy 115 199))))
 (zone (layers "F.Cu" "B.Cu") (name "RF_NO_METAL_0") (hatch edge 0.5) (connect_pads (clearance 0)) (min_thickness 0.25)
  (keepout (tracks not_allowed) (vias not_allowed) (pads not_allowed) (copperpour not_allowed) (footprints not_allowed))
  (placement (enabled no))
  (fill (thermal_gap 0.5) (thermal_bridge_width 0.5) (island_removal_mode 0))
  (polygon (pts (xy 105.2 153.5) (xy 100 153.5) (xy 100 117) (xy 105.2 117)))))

